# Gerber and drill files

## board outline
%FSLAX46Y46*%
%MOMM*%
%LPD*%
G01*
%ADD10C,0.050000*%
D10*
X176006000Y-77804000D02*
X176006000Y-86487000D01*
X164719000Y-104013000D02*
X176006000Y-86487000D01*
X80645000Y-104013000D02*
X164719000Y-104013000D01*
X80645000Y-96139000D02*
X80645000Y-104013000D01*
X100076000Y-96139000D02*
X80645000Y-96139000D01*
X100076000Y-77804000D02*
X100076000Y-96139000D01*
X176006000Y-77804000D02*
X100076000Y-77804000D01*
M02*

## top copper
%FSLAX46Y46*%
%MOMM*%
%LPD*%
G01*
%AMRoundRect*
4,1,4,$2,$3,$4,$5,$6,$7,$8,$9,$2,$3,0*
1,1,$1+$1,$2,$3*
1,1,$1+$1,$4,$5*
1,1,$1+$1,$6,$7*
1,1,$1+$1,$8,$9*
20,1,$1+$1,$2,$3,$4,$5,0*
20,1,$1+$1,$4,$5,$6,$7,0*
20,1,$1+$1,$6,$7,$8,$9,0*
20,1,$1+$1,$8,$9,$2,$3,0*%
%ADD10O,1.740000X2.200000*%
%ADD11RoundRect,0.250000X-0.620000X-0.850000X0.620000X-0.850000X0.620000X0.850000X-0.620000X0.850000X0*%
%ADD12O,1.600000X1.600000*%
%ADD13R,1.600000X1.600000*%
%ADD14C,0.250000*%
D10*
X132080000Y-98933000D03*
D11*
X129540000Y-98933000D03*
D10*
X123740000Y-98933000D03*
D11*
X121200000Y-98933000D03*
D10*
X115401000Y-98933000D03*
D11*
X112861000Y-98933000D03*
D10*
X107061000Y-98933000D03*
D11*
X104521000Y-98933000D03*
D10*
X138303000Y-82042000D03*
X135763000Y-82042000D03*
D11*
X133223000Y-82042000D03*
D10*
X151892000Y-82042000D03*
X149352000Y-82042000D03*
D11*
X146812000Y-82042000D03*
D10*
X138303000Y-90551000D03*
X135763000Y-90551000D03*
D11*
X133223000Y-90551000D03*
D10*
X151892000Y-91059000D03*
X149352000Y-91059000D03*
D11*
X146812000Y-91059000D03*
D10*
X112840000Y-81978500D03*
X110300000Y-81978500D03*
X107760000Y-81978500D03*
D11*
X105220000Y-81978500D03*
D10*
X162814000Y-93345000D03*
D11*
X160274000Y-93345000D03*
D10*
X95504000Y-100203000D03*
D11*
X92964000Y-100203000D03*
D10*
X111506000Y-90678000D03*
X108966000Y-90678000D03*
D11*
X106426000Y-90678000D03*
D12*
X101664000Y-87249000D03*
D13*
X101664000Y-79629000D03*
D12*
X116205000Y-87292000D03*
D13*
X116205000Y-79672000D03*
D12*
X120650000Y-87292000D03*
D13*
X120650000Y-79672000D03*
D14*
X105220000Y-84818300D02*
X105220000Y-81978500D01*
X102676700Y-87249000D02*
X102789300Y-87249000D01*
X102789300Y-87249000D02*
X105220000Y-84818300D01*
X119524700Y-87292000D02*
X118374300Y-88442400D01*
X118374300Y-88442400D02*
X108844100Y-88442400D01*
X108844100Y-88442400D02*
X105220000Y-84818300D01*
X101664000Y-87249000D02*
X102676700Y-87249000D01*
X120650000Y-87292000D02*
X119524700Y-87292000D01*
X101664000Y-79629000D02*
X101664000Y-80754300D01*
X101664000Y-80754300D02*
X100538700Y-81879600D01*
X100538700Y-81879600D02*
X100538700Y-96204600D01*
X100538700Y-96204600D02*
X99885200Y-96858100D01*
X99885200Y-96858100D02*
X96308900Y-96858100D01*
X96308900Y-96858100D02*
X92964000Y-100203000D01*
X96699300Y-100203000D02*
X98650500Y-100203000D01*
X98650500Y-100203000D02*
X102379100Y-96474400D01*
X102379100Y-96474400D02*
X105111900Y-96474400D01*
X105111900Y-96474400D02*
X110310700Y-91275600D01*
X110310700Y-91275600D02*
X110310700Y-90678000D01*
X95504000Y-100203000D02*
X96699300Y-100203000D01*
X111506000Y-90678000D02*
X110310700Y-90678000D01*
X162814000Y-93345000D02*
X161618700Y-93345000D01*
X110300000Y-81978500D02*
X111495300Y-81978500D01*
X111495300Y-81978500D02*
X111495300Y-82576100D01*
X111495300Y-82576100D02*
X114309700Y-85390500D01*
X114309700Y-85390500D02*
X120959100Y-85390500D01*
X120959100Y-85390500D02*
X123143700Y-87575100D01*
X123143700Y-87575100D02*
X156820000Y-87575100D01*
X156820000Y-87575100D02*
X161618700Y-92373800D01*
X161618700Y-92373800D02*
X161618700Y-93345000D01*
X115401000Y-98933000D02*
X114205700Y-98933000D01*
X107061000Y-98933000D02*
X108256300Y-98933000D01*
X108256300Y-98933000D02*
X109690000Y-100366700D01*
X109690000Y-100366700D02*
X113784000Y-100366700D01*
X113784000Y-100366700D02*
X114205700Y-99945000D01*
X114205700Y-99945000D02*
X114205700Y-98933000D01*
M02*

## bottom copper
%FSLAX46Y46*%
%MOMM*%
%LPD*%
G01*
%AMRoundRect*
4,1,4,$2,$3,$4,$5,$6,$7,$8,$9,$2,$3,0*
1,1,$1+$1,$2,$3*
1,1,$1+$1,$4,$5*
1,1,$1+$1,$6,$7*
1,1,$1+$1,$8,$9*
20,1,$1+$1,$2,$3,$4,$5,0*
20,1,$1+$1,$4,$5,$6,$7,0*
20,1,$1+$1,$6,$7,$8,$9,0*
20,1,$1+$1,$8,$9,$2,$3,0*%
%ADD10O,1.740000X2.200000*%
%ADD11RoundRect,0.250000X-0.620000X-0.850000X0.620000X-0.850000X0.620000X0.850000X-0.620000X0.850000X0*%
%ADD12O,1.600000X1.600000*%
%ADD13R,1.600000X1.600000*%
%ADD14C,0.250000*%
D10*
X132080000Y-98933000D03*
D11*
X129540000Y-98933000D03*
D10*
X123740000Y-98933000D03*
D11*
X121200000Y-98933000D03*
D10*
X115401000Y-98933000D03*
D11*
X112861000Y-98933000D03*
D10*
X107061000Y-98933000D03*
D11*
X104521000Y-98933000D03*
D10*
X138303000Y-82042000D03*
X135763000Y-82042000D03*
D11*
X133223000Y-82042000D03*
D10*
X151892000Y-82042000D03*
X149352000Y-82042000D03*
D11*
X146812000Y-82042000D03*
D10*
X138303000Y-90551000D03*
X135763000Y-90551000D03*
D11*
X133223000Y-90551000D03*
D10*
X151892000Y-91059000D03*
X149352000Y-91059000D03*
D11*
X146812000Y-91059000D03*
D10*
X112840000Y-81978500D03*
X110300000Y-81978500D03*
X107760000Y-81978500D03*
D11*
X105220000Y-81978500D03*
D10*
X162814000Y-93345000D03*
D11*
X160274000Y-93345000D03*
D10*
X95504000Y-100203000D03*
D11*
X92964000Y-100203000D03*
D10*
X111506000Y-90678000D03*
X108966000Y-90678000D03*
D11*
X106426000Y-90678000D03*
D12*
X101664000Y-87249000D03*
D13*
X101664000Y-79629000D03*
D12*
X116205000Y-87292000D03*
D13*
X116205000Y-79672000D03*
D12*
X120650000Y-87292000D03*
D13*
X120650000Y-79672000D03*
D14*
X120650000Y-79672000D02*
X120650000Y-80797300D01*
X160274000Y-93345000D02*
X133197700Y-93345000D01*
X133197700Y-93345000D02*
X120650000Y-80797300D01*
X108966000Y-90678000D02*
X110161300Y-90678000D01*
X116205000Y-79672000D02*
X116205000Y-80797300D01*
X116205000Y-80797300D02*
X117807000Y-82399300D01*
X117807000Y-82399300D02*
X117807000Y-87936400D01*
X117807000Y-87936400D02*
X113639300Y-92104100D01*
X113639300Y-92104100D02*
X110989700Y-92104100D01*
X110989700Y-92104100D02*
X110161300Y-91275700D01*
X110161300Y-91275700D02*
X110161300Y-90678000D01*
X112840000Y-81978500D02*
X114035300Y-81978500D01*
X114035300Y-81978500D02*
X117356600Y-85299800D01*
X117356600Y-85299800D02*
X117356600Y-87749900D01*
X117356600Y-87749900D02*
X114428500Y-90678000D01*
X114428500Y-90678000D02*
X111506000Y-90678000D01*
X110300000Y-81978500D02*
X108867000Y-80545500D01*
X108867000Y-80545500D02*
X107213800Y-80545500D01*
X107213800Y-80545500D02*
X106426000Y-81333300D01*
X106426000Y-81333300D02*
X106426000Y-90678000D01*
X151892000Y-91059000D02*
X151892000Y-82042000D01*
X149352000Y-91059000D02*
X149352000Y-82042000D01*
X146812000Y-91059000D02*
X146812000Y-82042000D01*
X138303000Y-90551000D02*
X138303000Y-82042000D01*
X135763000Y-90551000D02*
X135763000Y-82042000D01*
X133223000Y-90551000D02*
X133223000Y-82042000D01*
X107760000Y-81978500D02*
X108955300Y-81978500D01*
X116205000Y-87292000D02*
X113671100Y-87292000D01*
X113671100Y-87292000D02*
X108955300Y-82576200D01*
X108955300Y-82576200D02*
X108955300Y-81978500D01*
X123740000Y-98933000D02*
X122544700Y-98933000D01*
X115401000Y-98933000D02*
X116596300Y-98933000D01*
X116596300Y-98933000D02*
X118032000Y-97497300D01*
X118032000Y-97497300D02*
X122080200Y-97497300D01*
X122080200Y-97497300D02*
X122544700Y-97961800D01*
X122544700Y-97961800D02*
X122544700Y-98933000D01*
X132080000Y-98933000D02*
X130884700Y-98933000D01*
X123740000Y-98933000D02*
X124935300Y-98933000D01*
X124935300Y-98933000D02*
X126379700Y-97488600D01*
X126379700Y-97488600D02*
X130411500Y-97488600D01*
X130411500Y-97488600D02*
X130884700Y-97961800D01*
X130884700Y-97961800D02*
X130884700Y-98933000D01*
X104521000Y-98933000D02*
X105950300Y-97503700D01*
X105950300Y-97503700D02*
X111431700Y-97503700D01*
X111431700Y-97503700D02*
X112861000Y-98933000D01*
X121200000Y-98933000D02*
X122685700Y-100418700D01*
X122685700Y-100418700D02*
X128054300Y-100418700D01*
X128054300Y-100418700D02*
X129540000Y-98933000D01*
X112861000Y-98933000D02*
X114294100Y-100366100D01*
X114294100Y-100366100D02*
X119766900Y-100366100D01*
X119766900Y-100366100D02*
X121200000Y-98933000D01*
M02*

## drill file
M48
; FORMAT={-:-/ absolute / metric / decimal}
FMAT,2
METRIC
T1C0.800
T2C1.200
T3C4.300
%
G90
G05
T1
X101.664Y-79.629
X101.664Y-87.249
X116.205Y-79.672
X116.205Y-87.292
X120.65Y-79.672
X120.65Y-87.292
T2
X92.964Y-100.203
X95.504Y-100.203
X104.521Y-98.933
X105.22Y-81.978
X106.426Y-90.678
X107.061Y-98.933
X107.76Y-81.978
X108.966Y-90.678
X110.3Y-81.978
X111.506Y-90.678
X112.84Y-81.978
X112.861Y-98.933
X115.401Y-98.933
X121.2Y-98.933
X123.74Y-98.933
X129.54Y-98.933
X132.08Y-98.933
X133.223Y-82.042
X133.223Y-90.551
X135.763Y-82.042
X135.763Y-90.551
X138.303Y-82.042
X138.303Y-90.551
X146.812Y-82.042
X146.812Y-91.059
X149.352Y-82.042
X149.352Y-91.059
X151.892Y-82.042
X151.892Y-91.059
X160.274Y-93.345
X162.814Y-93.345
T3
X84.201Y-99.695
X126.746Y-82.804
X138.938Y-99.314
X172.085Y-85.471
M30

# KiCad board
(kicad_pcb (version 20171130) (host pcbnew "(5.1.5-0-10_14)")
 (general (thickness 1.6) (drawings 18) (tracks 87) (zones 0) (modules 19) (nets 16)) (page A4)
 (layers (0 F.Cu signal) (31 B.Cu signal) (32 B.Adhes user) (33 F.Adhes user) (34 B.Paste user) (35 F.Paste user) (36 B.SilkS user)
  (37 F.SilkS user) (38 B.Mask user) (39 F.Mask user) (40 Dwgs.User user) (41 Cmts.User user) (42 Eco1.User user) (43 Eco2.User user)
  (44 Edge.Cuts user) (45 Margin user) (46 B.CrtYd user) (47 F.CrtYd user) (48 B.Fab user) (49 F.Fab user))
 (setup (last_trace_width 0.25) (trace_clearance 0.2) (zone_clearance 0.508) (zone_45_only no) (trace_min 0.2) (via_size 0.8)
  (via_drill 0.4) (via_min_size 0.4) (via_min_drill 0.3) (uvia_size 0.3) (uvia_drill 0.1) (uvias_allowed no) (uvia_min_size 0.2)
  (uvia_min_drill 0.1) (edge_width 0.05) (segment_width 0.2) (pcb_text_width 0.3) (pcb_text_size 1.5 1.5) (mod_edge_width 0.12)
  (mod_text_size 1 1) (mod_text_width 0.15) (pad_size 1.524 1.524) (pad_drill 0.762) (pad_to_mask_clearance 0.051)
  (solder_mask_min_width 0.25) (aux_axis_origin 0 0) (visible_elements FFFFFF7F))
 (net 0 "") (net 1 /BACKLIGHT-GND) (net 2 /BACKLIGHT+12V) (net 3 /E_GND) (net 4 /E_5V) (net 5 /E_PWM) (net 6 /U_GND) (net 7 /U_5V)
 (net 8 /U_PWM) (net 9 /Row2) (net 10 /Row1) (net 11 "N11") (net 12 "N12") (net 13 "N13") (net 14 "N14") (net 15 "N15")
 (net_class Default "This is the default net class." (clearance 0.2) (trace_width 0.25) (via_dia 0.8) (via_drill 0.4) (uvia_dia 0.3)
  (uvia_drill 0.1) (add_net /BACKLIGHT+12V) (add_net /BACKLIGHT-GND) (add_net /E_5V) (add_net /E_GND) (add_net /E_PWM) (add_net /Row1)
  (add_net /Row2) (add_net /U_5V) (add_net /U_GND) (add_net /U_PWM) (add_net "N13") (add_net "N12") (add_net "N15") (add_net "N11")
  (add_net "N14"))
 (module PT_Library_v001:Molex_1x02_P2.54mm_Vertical (layer F.Cu) (at 129.54 98.933)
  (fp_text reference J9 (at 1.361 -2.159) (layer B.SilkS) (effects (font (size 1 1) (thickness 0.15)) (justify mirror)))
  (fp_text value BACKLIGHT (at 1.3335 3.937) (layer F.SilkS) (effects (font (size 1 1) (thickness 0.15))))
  (pad 2 thru_hole oval (at 2.54 0) (size 1.74 2.2) (drill 1.2) (layers *.Cu *.Mask) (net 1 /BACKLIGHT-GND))
  (pad 1 thru_hole roundrect (at 0 0) (size 1.74 2.2) (drill 1.2) (layers *.Cu *.Mask) (roundrect_rratio 0.143678) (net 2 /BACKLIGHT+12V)))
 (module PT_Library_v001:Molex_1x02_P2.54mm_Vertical (layer F.Cu) (at 121.2 98.933)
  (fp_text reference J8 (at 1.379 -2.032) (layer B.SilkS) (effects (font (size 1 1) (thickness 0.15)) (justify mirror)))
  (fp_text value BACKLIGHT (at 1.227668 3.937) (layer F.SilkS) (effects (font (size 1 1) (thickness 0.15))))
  (pad 2 thru_hole oval (at 2.54 0) (size 1.74 2.2) (drill 1.2) (layers *.Cu *.Mask) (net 1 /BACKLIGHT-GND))
  (pad 1 thru_hole roundrect (at 0 0) (size 1.74 2.2) (drill 1.2) (layers *.Cu *.Mask) (roundrect_rratio 0.143678) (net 2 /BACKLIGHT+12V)))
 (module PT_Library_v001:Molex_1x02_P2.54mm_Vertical (layer F.Cu) (at 112.861 98.933)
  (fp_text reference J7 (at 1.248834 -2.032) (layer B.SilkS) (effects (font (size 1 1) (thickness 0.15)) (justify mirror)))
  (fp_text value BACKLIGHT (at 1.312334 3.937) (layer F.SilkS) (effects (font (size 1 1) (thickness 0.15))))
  (pad 2 thru_hole oval (at 2.54 0) (size 1.74 2.2) (drill 1.2) (layers *.Cu *.Mask) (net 1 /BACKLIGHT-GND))
  (pad 1 thru_hole roundrect (at 0 0) (size 1.74 2.2) (drill 1.2) (layers *.Cu *.Mask) (roundrect_rratio 0.143678) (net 2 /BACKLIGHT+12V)))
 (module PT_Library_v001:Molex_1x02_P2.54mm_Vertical (layer F.Cu) (at 104.521 98.933)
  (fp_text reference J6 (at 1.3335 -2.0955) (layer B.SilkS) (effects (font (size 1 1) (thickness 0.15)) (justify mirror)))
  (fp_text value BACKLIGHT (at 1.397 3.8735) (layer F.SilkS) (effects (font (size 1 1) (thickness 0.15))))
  (pad 2 thru_hole oval (at 2.54 0) (size 1.74 2.2) (drill 1.2) (layers *.Cu *.Mask) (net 1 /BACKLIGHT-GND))
  (pad 1 thru_hole roundrect (at 0 0) (size 1.74 2.2) (drill 1.2) (layers *.Cu *.Mask) (roundrect_rratio 0.143678) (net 2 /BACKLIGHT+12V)))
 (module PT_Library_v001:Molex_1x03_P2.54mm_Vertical (layer F.Cu) (at 133.223 82.042)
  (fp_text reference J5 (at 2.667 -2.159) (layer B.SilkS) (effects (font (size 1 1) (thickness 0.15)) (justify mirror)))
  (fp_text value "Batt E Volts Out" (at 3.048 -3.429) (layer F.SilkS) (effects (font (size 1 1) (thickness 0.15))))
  (pad 3 thru_hole oval (at 5.08 0) (size 1.74 2.2) (drill 1.2) (layers *.Cu *.Mask) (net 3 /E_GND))
  (pad 2 thru_hole oval (at 2.54 0) (size 1.74 2.2) (drill 1.2) (layers *.Cu *.Mask) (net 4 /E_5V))
  (pad 1 thru_hole roundrect (at 0 0) (size 1.74 2.2) (drill 1.2) (layers *.Cu *.Mask) (roundrect_rratio 0.143678) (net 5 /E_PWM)))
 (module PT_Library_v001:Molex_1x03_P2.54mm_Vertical (layer F.Cu) (at 146.812 82.042)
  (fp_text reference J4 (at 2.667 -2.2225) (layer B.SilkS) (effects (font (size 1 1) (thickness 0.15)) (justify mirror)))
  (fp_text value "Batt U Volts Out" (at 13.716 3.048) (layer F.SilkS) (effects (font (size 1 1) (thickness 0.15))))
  (pad 3 thru_hole oval (at 5.08 0) (size 1.74 2.2) (drill 1.2) (layers *.Cu *.Mask) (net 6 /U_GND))
  (pad 2 thru_hole oval (at 2.54 0) (size 1.74 2.2) (drill 1.2) (layers *.Cu *.Mask) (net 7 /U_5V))
  (pad 1 thru_hole roundrect (at 0 0) (size 1.74 2.2) (drill 1.2) (layers *.Cu *.Mask) (roundrect_rratio 0.143678) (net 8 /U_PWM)))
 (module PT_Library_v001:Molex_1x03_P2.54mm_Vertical (layer F.Cu) (at 133.223 90.551)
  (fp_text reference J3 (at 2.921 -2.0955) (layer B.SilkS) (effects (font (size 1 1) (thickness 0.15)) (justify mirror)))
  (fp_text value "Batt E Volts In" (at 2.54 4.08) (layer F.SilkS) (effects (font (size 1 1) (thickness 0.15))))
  (pad 3 thru_hole oval (at 5.08 0) (size 1.74 2.2) (drill 1.2) (layers *.Cu *.Mask) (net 3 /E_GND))
  (pad 2 thru_hole oval (at 2.54 0) (size 1.74 2.2) (drill 1.2) (layers *.Cu *.Mask) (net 4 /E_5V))
  (pad 1 thru_hole roundrect (at 0 0) (size 1.74 2.2) (drill 1.2) (layers *.Cu *.Mask) (roundrect_rratio 0.143678) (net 5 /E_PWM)))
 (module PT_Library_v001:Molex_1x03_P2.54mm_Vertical (layer F.Cu) (at 146.812 91.059)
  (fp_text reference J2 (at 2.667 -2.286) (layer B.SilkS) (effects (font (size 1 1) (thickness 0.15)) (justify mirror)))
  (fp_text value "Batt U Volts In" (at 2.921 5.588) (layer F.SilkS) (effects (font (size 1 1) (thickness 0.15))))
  (pad 3 thru_hole oval (at 5.08 0) (size 1.74 2.2) (drill 1.2) (layers *.Cu *.Mask) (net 6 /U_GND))
  (pad 2 thru_hole oval (at 2.54 0) (size 1.74 2.2) (drill 1.2) (layers *.Cu *.Mask) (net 7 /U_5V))
  (pad 1 thru_hole roundrect (at 0 0) (size 1.74 2.2) (drill 1.2) (layers *.Cu *.Mask) (roundrect_rratio 0.143678) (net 8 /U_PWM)))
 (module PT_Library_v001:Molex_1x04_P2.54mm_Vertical (layer F.Cu) (at 105.22 81.9785)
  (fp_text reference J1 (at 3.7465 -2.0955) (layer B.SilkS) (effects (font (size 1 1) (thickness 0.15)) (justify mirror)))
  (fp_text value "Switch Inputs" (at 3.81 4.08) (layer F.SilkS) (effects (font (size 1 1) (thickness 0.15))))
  (pad 4 thru_hole oval (at 7.62 0) (size 1.74 2.2) (drill 1.2) (layers *.Cu *.Mask) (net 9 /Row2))
  (pad 3 thru_hole oval (at 5.08 0) (size 1.74 2.2) (drill 1.2) (layers *.Cu *.Mask) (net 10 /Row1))
  (pad 2 thru_hole oval (at 2.54 0) (size 1.74 2.2) (drill 1.2) (layers *.Cu *.Mask) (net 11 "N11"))
  (pad 1 thru_hole roundrect (at 0 0) (size 1.74 2.2) (drill 1.2) (layers *.Cu *.Mask) (roundrect_rratio 0.143678) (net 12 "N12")))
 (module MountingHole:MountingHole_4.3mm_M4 (layer F.Cu) (at 172.085 85.471)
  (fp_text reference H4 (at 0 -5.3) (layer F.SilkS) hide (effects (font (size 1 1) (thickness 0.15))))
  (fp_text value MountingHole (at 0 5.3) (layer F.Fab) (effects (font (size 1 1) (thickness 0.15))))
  (pad 1 np_thru_hole circle (at 0 0) (size 4.3 4.3) (drill 4.3) (layers *.Cu *.Mask)))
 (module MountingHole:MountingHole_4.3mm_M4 (layer F.Cu) (at 126.746 82.804)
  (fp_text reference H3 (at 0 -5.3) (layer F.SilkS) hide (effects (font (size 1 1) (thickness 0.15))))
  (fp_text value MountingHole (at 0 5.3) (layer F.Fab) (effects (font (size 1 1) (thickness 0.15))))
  (pad 1 np_thru_hole circle (at 0 0) (size 4.3 4.3) (drill 4.3) (layers *.Cu *.Mask)))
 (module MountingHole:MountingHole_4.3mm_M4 (layer F.Cu) (at 84.201 99.695)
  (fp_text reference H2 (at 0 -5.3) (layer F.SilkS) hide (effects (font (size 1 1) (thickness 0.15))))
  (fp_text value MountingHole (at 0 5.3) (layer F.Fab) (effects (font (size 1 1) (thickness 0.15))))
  (pad 1 np_thru_hole circle (at 0 0) (size 4.3 4.3) (drill 4.3) (layers *.Cu *.Mask)))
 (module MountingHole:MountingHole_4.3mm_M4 (layer F.Cu) (at 138.938 99.314)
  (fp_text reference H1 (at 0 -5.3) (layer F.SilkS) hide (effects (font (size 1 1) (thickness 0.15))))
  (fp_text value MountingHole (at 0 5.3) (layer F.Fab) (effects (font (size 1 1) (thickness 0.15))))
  (pad 1 np_thru_hole circle (at 0 0) (size 4.3 4.3) (drill 4.3) (layers *.Cu *.Mask)))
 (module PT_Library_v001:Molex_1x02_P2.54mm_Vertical (layer F.Cu) (at 160.274 93.345)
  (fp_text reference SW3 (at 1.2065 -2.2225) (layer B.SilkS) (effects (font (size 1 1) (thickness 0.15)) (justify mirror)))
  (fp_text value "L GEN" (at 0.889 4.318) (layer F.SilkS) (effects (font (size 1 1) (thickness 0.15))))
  (pad 2 thru_hole oval (at 2.54 0) (size 1.74 2.2) (drill 1.2) (layers *.Cu *.Mask) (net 10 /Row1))
  (pad 1 thru_hole roundrect (at 0 0) (size 1.74 2.2) (drill 1.2) (layers *.Cu *.Mask) (roundrect_rratio 0.143678) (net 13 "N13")))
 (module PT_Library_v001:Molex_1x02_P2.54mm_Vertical (layer F.Cu) (at 92.964 100.203)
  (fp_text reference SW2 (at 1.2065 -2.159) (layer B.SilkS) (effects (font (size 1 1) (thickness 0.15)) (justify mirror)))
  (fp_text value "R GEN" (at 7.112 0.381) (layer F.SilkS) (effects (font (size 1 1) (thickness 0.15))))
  (pad 2 thru_hole oval (at 2.54 0) (size 1.74 2.2) (drill 1.2) (layers *.Cu *.Mask) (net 9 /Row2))
  (pad 1 thru_hole roundrect (at 0 0) (size 1.74 2.2) (drill 1.2) (layers *.Cu *.Mask) (roundrect_rratio 0.143678) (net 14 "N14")))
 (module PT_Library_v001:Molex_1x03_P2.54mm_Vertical (layer F.Cu) (at 106.426 90.678)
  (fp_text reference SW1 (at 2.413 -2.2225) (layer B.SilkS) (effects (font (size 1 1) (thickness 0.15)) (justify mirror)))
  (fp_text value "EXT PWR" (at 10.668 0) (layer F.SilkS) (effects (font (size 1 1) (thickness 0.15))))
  (pad 3 thru_hole oval (at 5.08 0) (size 1.74 2.2) (drill 1.2) (layers *.Cu *.Mask) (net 9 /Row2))
  (pad 2 thru_hole oval (at 2.54 0) (size 1.74 2.2) (drill 1.2) (layers *.Cu *.Mask) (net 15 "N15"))
  (pad 1 thru_hole roundrect (at 0 0) (size 1.74 2.2) (drill 1.2) (layers *.Cu *.Mask) (roundrect_rratio 0.143678) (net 10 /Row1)))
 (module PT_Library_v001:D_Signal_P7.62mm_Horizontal (layer F.Cu) (at 101.664 79.629 270)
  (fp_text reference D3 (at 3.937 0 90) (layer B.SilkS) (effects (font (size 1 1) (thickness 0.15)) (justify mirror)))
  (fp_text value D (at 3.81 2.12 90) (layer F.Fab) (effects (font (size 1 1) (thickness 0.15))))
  (pad 2 thru_hole oval (at 7.62 0 270) (size 1.6 1.6) (drill 0.8) (layers *.Cu *.Mask) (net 12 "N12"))
  (pad 1 thru_hole rect (at 0 0 270) (size 1.6 1.6) (drill 0.8) (layers *.Cu *.Mask) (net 14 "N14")))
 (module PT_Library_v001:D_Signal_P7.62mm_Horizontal (layer F.Cu) (at 116.205 79.672 270)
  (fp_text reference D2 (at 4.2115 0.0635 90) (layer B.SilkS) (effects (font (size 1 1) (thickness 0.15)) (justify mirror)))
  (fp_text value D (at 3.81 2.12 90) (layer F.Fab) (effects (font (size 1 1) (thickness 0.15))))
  (pad 2 thru_hole oval (at 7.62 0 270) (size 1.6 1.6) (drill 0.8) (layers *.Cu *.Mask) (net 11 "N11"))
  (pad 1 thru_hole rect (at 0 0 270) (size 1.6 1.6) (drill 0.8) (layers *.Cu *.Mask) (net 15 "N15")))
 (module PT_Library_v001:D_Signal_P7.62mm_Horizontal (layer F.Cu) (at 120.65 79.672 270)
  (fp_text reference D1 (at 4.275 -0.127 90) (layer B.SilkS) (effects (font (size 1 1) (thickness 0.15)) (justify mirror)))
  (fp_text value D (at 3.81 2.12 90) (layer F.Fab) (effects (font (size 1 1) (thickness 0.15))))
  (pad 2 thru_hole oval (at 7.62 0 270) (size 1.6 1.6) (drill 0.8) (layers *.Cu *.Mask) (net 12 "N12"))
  (pad 1 thru_hole rect (at 0 0 270) (size 1.6 1.6) (drill 0.8) (layers *.Cu *.Mask) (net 13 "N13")))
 (gr_line (start 176.006 77.804) (end 176.006 86.487) (layer Edge.Cuts) (width 0.05))
 (gr_line (start 164.719 104.013) (end 176.006 86.487) (layer Edge.Cuts) (width 0.05))
 (gr_line (start 80.645 104.013) (end 164.719 104.013) (layer Edge.Cuts) (width 0.05))
 (gr_line (start 80.645 96.139) (end 80.645 104.013) (layer Edge.Cuts) (width 0.05))
 (gr_line (start 100.076 96.139) (end 80.645 96.139) (layer Edge.Cuts) (width 0.05))
 (gr_line (start 100.076 77.804) (end 100.076 96.139) (layer Edge.Cuts) (width 0.05))
 (gr_line (start 176.006 77.804) (end 100.076 77.804) (layer Edge.Cuts) (width 0.05))
 (segment (start 105.22 84.8183) (end 105.22 81.9785) (width 0.25) (layer F.Cu) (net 12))
 (segment (start 102.6767 87.249) (end 102.7893 87.249) (width 0.25) (layer F.Cu) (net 12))
 (segment (start 102.7893 87.249) (end 105.22 84.8183) (width 0.25) (layer F.Cu) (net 12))
 (segment (start 119.5247 87.292) (end 118.3743 88.4424) (width 0.25) (layer F.Cu) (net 12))
 (segment (start 118.3743 88.4424) (end 108.8441 88.4424) (width 0.25) (layer F.Cu) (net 12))
 (segment (start 108.8441 88.4424) (end 105.22 84.8183) (width 0.25) (layer F.Cu) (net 12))
 (segment (start 101.664 87.249) (end 102.6767 87.249) (width 0.25) (layer F.Cu) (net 12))
 (segment (start 120.65 87.292) (end 119.5247 87.292) (width 0.25) (layer F.Cu) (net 12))
 (segment (start 120.65 79.672) (end 120.65 80.7973) (width 0.25) (layer B.Cu) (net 13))
 (segment (start 160.274 93.345) (end 133.1977 93.345) (width 0.25) (layer B.Cu) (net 13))
 (segment (start 133.1977 93.345) (end 120.65 80.7973) (width 0.25) (layer B.Cu) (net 13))
 (segment (start 108.966 90.678) (end 110.1613 90.678) (width 0.25) (layer B.Cu) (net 15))
 (segment (start 116.205 79.672) (end 116.205 80.7973) (width 0.25) (layer B.Cu) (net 15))
 (segment (start 116.205 80.7973) (end 117.807 82.3993) (width 0.25) (layer B.Cu) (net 15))
 (segment (start 117.807 82.3993) (end 117.807 87.9364) (width 0.25) (layer B.Cu) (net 15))
 (segment (start 117.807 87.9364) (end 113.6393 92.1041) (width 0.25) (layer B.Cu) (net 15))
 (segment (start 113.6393 92.1041) (end 110.9897 92.1041) (width 0.25) (layer B.Cu) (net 15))
 (segment (start 110.9897 92.1041) (end 110.1613 91.2757) (width 0.25) (layer B.Cu) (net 15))
 (segment (start 110.1613 91.2757) (end 110.1613 90.678) (width 0.25) (layer B.Cu) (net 15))
 (segment (start 101.664 79.629) (end 101.664 80.7543) (width 0.25) (layer F.Cu) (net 14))
 (segment (start 101.664 80.7543) (end 100.5387 81.8796) (width 0.25) (layer F.Cu) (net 14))
 (segment (start 100.5387 81.8796) (end 100.5387 96.2046) (width 0.25) (layer F.Cu) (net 14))
 (segment (start 100.5387 96.2046) (end 99.8852 96.8581) (width 0.25) (layer F.Cu) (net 14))
 (segment (start 99.8852 96.8581) (end 96.3089 96.8581) (width 0.25) (layer F.Cu) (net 14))
 (segment (start 96.3089 96.8581) (end 92.964 100.203) (width 0.25) (layer F.Cu) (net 14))
 (segment (start 96.6993 100.203) (end 98.6505 100.203) (width 0.25) (layer F.Cu) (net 9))
 (segment (start 98.6505 100.203) (end 102.3791 96.4744) (width 0.25) (layer F.Cu) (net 9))
 (segment (start 102.3791 96.4744) (end 105.1119 96.4744) (width 0.25) (layer F.Cu) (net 9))
 (segment (start 105.1119 96.4744) (end 110.3107 91.2756) (width 0.25) (layer F.Cu) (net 9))
 (segment (start 110.3107 91.2756) (end 110.3107 90.678) (width 0.25) (layer F.Cu) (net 9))
 (segment (start 112.84 81.9785) (end 114.0353 81.9785) (width 0.25) (layer B.Cu) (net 9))
 (segment (start 114.0353 81.9785) (end 117.3566 85.2998) (width 0.25) (layer B.Cu) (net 9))
 (segment (start 117.3566 85.2998) (end 117.3566 87.7499) (width 0.25) (layer B.Cu) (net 9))
 (segment (start 117.3566 87.7499) (end 114.4285 90.678) (width 0.25) (layer B.Cu) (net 9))
 (segment (start 114.4285 90.678) (end 111.506 90.678) (width 0.25) (layer B.Cu) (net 9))
 (segment (start 95.504 100.203) (end 96.6993 100.203) (width 0.25) (layer F.Cu) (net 9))
 (segment (start 111.506 90.678) (end 110.3107 90.678) (width 0.25) (layer F.Cu) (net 9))
 (segment (start 162.814 93.345) (end 161.6187 93.345) (width 0.25) (layer F.Cu) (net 10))
 (segment (start 110.3 81.9785) (end 111.4953 81.9785) (width 0.25) (layer F.Cu) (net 10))
 (segment (start 111.4953 81.9785) (end 111.4953 82.5761) (width 0.25) (layer F.Cu) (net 10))
 (segment (start 111.4953 82.5761) (end 114.3097 85.3905) (width 0.25) (layer F.Cu) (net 10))
 (segment (start 114.3097 85.3905) (end 120.9591 85.3905) (width 0.25) (layer F.Cu) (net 10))
 (segment (start 120.9591 85.3905) (end 123.1437 87.5751) (width 0.25) (layer F.Cu) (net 10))
 (segment (start 123.1437 87.5751) (end 156.82 87.5751) (width 0.25) (layer F.Cu) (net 10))
 (segment (start 156.82 87.5751) (end 161.6187 92.3738) (width 0.25) (layer F.Cu) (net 10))
 (segment (start 161.6187 92.3738) (end 161.6187 93.345) (width 0.25) (layer F.Cu) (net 10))
 (segment (start 110.3 81.9785) (end 108.867 80.5455) (width 0.25) (layer B.Cu) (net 10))
 (segment (start 108.867 80.5455) (end 107.2138 80.5455) (width 0.25) (layer B.Cu) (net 10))
 (segment (start 107.2138 80.5455) (end 106.426 81.3333) (width 0.25) (layer B.Cu) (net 10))
 (segment (start 106.426 81.3333) (end 106.426 90.678) (width 0.25) (layer B.Cu) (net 10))
 (segment (start 151.892 91.059) (end 151.892 82.042) (width 0.25) (layer B.Cu) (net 6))
 (segment (start 149.352 91.059) (end 149.352 82.042) (width 0.25) (layer B.Cu) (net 7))
 (segment (start 146.812 91.059) (end 146.812 82.042) (width 0.25) (layer B.Cu) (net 8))
 (segment (start 138.303 90.551) (end 138.303 82.042) (width 0.25) (layer B.Cu) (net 3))
 (segment (start 135.763 90.551) (end 135.763 82.042) (width 0.25) (layer B.Cu) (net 4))
 (segment (start 133.223 90.551) (end 133.223 82.042) (width 0.25) (layer B.Cu) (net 5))
 (segment (start 107.76 81.9785) (end 108.9553 81.9785) (width 0.25) (layer B.Cu) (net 11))
 (segment (start 116.205 87.292) (end 113.6711 87.292) (width 0.25) (layer B.Cu) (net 11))
 (segment (start 113.6711 87.292) (end 108.9553 82.5762) (width 0.25) (layer B.Cu) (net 11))
 (segment (start 108.9553 82.5762) (end 108.9553 81.9785) (width 0.25) (layer B.Cu) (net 11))
 (segment (start 123.74 98.933) (end 122.5447 98.933) (width 0.25) (layer B.Cu) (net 1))
 (segment (start 115.401 98.933) (end 116.5963 98.933) (width 0.25) (layer B.Cu) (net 1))
 (segment (start 116.5963 98.933) (end 118.032 97.4973) (width 0.25) (layer B.Cu) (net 1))
 (segment (start 118.032 97.4973) (end 122.0802 97.4973) (width 0.25) (layer B.Cu) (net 1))
 (segment (start 122.0802 97.4973) (end 122.5447 97.9618) (width 0.25) (layer B.Cu) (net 1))
 (segment (start 122.5447 97.9618) (end 122.5447 98.933) (width 0.25) (layer B.Cu) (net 1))
 (segment (start 115.401 98.933) (end 114.2057 98.933) (width 0.25) (layer F.Cu) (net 1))
 (segment (start 107.061 98.933) (end 108.2563 98.933) (width 0.25) (layer F.Cu) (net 1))
 (segment (start 108.2563 98.933) (end 109.69 100.3667) (width 0.25) (layer F.Cu) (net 1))
 (segment (start 109.69 100.3667) (end 113.784 100.3667) (width 0.25) (layer F.Cu) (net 1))
 (segment (start 113.784 100.3667) (end 114.2057 99.945) (width 0.25) (layer F.Cu) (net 1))
 (segment (start 114.2057 99.945) (end 114.2057 98.933) (width 0.25) (layer F.Cu) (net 1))
 (segment (start 132.08 98.933) (end 130.8847 98.933) (width 0.25) (layer B.Cu) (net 1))
 (segment (start 123.74 98.933) (end 124.9353 98.933) (width 0.25) (layer B.Cu) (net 1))
 (segment (start 124.9353 98.933) (end 126.3797 97.4886) (width 0.25) (layer B.Cu) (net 1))
 (segment (start 126.3797 97.4886) (end 130.4115 97.4886) (width 0.25) (layer B.Cu) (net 1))
 (segment (start 130.4115 97.4886) (end 130.8847 97.9618) (width 0.25) (layer B.Cu) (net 1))
 (segment (start 130.8847 97.9618) (end 130.8847 98.933) (width 0.25) (layer B.Cu) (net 1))
 (segment (start 104.521 98.933) (end 105.9503 97.5037) (width 0.25) (layer B.Cu) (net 2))
 (segment (start 105.9503 97.5037) (end 111.4317 97.5037) (width 0.25) (layer B.Cu) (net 2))
 (segment (start 111.4317 97.5037) (end 112.861 98.933) (width 0.25) (layer B.Cu) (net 2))
 (segment (start 121.2 98.933) (end 122.6857 100.4187) (width 0.25) (layer B.Cu) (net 2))
 (segment (start 122.6857 100.4187) (end 128.0543 100.4187) (width 0.25) (layer B.Cu) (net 2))
 (segment (start 128.0543 100.4187) (end 129.54 98.933) (width 0.25) (layer B.Cu) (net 2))
 (segment (start 112.861 98.933) (end 114.2941 100.3661) (width 0.25) (layer B.Cu) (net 2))
 (segment (start 114.2941 100.3661) (end 119.7669 100.3661) (width 0.25) (layer B.Cu) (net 2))
 (segment (start 119.7669 100.3661) (end 121.2 98.933) (width 0.25) (layer B.Cu) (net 2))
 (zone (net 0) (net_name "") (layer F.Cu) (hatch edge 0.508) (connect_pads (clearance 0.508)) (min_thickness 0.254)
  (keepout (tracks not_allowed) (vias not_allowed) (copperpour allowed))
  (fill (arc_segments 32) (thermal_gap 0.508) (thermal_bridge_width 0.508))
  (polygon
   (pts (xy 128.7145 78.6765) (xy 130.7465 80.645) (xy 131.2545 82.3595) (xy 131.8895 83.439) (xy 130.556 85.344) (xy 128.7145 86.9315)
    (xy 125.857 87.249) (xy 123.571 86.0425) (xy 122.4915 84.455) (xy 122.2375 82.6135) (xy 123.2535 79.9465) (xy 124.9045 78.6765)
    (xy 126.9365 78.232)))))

